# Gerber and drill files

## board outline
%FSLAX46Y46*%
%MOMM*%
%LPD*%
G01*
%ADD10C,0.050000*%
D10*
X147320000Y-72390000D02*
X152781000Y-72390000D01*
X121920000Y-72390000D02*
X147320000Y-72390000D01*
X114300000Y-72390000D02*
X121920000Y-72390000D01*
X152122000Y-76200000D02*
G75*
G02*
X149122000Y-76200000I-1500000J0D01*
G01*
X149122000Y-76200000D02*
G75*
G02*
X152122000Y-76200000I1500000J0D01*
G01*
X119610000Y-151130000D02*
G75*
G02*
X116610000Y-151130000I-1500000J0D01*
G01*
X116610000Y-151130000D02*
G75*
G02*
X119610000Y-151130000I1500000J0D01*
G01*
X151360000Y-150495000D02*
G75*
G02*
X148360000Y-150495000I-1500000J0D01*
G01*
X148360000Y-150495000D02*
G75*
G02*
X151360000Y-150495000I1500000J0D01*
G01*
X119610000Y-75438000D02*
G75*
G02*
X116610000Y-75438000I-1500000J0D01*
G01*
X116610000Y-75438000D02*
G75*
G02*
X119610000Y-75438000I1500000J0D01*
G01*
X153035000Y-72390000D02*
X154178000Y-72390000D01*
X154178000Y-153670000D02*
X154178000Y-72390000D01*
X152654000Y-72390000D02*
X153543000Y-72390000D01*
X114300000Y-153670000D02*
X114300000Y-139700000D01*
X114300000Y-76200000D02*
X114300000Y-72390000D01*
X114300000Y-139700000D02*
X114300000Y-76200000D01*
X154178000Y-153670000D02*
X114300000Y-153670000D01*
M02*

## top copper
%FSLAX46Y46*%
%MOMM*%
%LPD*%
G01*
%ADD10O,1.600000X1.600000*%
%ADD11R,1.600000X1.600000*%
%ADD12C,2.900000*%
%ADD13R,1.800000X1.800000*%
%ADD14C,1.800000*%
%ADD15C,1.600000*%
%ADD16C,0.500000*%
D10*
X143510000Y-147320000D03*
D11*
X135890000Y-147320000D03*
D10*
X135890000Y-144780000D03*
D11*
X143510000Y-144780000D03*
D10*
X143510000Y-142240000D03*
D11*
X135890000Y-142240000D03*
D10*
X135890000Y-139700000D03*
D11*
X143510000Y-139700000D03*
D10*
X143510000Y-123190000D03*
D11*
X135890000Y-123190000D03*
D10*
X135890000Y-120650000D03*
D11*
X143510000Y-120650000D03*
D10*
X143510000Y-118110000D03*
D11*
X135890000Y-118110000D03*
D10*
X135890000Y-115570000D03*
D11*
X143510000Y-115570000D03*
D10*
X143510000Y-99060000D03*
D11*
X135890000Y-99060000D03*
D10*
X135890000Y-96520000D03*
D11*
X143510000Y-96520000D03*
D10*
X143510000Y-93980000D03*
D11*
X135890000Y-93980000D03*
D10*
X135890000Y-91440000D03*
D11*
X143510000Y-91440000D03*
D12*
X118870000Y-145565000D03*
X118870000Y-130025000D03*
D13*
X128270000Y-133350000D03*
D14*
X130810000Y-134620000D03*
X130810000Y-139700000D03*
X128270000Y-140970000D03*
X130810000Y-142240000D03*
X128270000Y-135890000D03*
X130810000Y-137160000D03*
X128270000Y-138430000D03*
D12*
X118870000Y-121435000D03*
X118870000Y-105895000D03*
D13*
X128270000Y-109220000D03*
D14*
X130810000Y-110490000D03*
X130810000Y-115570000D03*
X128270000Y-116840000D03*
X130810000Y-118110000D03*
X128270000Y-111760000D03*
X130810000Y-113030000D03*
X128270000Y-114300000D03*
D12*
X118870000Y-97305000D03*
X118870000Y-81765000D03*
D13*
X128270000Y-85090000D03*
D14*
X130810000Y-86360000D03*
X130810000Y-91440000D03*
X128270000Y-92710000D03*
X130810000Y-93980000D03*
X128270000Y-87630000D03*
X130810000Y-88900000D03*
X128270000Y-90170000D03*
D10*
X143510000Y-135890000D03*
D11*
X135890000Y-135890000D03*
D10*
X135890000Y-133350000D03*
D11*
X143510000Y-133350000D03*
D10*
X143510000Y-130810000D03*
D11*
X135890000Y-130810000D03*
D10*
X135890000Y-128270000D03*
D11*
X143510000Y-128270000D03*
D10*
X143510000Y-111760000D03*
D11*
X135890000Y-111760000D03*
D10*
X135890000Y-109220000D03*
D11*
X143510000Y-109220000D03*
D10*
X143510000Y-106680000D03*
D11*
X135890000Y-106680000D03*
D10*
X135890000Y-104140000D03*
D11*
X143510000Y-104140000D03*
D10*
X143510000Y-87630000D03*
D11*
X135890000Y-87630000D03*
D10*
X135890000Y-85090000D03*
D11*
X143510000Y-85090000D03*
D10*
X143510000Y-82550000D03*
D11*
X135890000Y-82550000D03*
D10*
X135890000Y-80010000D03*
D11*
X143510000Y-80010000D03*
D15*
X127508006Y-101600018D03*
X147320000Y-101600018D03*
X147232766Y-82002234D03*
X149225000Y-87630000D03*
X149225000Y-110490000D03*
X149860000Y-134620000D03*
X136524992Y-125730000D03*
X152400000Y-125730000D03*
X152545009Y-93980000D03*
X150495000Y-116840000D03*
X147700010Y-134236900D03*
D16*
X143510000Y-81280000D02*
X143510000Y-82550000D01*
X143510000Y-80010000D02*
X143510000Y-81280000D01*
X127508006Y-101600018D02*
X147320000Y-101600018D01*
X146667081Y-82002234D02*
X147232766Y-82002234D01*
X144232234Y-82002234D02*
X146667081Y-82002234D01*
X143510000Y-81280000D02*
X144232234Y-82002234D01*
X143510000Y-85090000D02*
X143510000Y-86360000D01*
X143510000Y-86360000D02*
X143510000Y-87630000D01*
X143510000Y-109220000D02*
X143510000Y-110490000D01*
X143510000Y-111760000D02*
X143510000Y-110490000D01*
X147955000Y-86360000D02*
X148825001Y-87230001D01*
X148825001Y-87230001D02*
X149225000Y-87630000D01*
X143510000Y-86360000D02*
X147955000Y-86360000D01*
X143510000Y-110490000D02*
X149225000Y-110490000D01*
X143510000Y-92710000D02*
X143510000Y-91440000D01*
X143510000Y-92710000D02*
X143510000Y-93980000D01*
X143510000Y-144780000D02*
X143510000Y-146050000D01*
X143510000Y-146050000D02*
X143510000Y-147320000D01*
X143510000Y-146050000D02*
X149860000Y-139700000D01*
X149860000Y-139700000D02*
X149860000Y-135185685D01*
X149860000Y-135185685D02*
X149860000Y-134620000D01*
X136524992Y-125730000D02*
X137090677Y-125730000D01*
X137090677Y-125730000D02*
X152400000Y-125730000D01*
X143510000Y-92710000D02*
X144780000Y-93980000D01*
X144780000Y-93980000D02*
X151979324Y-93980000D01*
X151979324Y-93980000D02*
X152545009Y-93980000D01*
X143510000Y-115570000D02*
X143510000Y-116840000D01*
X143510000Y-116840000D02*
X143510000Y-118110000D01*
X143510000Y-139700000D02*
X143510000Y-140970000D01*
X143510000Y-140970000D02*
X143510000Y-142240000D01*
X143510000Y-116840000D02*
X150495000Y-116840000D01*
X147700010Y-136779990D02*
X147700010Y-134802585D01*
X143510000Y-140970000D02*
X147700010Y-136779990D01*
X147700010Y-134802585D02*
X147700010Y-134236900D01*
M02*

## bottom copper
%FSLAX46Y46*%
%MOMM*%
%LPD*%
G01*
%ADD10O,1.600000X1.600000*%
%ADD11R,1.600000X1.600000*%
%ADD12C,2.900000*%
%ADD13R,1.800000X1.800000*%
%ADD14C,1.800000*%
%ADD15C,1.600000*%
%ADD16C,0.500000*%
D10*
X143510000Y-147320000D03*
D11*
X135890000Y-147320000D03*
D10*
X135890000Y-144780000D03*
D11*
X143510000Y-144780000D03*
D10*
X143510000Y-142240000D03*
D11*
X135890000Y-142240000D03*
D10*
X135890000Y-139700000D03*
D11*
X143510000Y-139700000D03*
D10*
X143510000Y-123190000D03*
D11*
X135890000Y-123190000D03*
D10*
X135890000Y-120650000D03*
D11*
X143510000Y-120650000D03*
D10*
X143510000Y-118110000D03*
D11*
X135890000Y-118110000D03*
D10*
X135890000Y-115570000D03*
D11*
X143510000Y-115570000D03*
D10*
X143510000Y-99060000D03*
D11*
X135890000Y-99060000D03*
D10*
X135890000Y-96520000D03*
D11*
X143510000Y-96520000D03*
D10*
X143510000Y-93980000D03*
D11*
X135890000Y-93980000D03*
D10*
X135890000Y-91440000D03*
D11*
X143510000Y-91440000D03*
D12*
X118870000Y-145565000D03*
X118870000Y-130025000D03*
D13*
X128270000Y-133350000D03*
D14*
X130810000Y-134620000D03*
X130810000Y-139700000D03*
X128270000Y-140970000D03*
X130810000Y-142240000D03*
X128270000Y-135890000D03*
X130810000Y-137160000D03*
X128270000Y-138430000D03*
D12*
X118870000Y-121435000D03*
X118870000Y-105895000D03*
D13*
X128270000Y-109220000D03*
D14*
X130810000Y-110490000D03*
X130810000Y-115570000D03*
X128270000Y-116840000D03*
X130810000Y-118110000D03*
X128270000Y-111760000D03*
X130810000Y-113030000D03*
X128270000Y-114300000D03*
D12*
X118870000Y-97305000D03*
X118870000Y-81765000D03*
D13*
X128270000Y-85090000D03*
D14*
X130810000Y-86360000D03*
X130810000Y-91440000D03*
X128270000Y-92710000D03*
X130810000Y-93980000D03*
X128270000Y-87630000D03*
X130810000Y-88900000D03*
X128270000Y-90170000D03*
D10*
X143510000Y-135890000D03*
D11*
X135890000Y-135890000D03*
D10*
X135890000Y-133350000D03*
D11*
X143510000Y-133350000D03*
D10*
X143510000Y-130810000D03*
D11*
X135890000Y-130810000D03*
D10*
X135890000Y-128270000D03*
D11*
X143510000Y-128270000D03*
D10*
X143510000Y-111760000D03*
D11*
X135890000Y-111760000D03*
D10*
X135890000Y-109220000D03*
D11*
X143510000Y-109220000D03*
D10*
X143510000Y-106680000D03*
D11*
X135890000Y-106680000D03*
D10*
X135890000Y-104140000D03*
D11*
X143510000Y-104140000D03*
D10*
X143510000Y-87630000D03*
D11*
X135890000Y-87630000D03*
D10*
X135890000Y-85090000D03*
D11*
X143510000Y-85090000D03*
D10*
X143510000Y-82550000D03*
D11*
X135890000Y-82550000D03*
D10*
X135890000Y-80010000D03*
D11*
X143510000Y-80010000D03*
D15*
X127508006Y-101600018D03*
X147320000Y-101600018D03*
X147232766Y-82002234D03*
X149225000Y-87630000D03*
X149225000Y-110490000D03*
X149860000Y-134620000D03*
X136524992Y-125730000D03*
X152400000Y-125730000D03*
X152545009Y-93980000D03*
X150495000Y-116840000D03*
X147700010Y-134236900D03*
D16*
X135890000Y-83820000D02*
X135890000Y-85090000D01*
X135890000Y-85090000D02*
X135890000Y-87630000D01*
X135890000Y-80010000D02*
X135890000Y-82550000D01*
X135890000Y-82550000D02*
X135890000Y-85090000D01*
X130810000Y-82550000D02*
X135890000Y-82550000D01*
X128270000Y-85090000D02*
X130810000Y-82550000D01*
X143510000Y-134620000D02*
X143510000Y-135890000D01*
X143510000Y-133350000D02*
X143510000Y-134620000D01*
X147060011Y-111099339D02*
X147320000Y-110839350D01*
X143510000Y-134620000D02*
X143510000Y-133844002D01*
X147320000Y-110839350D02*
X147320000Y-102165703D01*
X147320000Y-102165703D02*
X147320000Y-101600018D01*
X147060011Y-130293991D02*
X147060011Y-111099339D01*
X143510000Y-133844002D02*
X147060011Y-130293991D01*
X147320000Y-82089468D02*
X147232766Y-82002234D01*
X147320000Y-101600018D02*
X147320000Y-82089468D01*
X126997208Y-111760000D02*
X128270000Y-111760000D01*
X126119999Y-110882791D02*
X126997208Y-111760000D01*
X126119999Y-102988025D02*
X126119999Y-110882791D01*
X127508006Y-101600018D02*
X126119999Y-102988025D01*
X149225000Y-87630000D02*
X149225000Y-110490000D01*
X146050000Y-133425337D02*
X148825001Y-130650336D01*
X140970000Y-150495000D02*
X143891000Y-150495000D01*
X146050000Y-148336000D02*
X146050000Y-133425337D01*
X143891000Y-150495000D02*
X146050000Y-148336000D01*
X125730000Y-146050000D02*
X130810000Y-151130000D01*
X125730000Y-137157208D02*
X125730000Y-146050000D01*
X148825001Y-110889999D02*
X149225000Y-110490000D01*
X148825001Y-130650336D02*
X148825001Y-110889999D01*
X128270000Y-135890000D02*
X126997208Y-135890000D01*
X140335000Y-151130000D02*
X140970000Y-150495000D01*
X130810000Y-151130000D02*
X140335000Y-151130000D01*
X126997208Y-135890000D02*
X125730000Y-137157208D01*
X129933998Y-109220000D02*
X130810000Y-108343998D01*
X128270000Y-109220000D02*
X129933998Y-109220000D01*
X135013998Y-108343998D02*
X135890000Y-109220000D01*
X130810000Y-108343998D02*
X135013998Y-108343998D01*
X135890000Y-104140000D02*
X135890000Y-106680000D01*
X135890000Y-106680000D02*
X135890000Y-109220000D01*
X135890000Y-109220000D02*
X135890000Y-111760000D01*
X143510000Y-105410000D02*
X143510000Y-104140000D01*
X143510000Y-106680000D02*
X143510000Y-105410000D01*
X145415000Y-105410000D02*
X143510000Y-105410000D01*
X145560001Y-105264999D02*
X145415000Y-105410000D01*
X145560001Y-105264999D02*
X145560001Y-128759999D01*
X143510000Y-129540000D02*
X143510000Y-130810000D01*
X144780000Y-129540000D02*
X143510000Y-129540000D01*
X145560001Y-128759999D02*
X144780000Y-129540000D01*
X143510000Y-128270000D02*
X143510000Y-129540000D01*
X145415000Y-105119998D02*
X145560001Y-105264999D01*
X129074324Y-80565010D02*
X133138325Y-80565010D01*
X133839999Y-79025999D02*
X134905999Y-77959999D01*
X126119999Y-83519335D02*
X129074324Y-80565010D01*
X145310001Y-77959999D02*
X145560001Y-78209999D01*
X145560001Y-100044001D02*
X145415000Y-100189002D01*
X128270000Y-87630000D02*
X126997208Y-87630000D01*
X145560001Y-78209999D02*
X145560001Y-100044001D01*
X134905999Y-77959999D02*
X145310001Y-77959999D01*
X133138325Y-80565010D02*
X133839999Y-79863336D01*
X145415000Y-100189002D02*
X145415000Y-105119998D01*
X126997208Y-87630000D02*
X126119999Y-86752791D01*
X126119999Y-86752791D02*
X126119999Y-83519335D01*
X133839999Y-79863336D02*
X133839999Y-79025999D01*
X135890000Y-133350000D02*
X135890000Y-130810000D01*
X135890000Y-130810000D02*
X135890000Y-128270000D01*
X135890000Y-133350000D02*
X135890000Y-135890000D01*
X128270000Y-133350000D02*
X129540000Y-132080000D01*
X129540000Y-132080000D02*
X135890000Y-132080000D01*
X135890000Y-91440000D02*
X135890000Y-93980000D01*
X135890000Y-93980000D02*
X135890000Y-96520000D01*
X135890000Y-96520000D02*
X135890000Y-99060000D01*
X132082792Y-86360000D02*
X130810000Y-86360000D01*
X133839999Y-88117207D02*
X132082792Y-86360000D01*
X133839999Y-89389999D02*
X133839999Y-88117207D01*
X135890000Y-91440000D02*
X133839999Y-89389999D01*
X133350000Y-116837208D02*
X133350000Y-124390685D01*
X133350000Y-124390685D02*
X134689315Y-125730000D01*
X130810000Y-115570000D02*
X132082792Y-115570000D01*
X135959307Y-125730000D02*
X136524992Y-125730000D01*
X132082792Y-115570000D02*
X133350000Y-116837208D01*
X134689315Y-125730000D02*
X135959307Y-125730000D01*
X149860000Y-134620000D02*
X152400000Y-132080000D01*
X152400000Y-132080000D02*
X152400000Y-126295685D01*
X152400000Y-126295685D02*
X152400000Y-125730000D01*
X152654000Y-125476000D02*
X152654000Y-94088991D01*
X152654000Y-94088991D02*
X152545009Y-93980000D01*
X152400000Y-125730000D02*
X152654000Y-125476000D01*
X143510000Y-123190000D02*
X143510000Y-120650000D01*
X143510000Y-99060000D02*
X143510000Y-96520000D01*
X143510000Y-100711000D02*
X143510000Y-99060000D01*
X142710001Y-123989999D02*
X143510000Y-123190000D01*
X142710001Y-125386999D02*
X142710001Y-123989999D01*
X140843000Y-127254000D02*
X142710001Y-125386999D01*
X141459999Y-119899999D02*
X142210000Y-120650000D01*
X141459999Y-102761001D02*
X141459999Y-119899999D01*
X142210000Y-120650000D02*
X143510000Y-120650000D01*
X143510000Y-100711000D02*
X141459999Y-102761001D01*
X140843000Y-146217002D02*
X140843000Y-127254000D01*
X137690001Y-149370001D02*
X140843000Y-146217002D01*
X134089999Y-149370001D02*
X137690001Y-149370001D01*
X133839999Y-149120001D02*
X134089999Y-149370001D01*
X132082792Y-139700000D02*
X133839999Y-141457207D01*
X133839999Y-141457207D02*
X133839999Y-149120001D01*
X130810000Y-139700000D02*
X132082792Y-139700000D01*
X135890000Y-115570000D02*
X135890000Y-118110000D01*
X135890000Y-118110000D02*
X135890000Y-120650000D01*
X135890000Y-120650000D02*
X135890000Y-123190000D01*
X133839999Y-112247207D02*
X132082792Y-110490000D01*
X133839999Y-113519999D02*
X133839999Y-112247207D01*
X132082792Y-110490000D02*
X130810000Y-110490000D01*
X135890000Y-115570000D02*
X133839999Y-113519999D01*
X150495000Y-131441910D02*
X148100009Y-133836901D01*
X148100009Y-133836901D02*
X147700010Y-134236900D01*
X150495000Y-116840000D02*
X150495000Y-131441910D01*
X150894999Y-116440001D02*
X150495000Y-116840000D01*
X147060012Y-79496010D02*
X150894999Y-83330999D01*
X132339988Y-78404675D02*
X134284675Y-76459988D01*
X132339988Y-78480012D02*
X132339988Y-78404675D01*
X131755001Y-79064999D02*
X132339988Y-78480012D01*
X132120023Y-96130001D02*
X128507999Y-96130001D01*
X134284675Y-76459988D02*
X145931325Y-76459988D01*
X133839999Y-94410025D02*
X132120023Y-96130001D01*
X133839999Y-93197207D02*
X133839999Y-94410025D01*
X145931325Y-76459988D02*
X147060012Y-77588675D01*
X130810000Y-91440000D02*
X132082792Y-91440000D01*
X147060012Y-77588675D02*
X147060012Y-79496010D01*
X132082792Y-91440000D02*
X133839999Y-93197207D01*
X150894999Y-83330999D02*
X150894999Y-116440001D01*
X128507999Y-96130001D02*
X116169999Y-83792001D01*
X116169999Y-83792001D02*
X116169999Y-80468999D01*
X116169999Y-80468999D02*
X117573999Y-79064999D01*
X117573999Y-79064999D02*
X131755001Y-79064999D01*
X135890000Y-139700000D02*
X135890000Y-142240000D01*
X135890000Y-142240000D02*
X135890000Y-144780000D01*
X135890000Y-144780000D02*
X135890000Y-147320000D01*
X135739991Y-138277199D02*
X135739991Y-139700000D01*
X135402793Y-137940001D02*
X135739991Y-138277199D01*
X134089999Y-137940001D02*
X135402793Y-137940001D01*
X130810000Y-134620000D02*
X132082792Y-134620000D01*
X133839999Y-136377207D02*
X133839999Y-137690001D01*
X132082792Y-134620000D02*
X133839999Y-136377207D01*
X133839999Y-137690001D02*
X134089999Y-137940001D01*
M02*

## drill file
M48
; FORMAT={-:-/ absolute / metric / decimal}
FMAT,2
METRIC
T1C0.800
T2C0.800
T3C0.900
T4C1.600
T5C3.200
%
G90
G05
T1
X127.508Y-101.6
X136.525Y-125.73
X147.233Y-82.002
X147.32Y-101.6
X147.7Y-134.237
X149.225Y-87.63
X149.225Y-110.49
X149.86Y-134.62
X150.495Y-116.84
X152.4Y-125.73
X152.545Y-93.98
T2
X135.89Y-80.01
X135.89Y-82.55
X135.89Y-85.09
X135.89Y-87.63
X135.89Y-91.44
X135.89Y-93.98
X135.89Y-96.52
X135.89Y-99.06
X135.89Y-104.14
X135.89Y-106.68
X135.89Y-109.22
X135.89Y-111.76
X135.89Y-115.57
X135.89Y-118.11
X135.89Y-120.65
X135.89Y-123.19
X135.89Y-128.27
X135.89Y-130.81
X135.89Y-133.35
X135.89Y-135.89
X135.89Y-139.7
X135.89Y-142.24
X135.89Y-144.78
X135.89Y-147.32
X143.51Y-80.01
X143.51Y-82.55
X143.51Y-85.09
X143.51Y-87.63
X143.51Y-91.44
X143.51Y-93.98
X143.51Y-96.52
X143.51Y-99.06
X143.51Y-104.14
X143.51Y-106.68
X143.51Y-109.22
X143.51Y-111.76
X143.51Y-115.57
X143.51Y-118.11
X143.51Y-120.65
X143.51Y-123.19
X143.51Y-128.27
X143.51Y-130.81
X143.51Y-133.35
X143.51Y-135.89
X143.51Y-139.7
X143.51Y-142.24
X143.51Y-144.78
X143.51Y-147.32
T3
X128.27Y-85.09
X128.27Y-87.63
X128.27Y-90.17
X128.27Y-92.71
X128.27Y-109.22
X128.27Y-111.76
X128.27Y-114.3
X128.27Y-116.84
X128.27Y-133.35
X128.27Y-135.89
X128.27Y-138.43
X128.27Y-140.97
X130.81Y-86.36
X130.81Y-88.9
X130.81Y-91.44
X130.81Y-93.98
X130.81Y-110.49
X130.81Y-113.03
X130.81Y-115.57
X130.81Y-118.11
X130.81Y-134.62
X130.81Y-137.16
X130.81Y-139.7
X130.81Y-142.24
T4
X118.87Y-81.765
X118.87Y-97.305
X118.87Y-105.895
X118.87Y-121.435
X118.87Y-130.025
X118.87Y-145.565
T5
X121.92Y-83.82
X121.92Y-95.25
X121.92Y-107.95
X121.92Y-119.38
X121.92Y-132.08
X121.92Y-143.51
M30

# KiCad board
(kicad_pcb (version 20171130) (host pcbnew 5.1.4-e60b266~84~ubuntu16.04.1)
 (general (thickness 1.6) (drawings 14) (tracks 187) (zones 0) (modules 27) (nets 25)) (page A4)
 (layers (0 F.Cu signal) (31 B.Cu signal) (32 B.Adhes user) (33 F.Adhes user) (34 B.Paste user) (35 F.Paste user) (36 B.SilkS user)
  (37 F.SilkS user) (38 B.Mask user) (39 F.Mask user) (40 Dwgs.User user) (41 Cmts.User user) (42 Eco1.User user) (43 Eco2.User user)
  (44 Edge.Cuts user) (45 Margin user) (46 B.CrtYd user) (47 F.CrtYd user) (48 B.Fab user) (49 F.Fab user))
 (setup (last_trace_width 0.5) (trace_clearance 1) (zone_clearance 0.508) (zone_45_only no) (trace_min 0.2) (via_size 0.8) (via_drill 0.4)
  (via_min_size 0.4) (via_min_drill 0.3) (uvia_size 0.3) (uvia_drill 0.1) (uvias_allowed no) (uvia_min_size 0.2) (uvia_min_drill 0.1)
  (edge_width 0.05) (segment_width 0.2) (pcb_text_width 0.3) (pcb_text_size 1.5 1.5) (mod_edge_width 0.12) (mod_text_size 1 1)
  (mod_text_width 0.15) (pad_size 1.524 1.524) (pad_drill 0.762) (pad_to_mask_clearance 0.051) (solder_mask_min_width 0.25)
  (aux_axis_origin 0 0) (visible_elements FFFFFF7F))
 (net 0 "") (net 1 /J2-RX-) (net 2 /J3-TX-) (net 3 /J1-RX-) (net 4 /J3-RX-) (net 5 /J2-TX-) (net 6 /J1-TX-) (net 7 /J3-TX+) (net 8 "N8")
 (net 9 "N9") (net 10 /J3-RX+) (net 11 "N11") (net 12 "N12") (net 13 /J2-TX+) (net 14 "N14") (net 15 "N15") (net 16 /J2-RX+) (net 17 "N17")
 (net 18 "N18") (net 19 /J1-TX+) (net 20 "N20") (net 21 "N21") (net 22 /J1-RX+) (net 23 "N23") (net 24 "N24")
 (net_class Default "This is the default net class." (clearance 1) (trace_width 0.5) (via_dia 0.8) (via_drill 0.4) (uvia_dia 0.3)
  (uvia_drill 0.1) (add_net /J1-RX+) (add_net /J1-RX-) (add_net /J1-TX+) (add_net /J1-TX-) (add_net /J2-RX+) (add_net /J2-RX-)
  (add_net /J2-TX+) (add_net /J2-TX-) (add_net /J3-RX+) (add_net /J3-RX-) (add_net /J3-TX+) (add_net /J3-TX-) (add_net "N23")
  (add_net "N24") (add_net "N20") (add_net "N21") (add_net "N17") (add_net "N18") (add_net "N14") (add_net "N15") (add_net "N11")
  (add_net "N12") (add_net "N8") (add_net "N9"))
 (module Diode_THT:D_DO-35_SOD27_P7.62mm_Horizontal (layer F.Cu) (at 135.89 147.32)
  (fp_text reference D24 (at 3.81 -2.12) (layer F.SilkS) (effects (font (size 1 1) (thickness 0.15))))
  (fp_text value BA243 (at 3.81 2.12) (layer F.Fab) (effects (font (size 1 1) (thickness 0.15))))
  (pad 2 thru_hole oval (at 7.62 0) (size 1.6 1.6) (drill 0.8) (layers *.Cu *.Mask) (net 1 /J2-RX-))
  (pad 1 thru_hole rect (at 0 0) (size 1.6 1.6) (drill 0.8) (layers *.Cu *.Mask) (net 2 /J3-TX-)))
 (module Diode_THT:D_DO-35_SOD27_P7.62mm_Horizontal (layer F.Cu) (at 143.51 144.78 180)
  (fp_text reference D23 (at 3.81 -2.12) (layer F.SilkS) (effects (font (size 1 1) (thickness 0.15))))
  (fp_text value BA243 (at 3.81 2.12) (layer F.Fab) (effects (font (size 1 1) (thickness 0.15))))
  (pad 2 thru_hole oval (at 7.62 0 180) (size 1.6 1.6) (drill 0.8) (layers *.Cu *.Mask) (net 2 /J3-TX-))
  (pad 1 thru_hole rect (at 0 0 180) (size 1.6 1.6) (drill 0.8) (layers *.Cu *.Mask) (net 1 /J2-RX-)))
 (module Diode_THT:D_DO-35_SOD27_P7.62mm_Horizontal (layer F.Cu) (at 135.89 142.24)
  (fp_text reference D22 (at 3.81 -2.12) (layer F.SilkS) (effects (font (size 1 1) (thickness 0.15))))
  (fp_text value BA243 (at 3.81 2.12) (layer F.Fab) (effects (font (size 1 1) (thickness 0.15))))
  (pad 2 thru_hole oval (at 7.62 0) (size 1.6 1.6) (drill 0.8) (layers *.Cu *.Mask) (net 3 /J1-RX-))
  (pad 1 thru_hole rect (at 0 0) (size 1.6 1.6) (drill 0.8) (layers *.Cu *.Mask) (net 2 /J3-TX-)))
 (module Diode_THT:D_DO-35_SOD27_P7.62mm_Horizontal (layer F.Cu) (at 143.51 139.7 180)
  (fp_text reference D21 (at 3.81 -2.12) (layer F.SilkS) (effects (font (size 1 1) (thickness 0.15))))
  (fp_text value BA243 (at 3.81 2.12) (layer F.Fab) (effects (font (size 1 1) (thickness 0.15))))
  (pad 2 thru_hole oval (at 7.62 0 180) (size 1.6 1.6) (drill 0.8) (layers *.Cu *.Mask) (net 2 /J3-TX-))
  (pad 1 thru_hole rect (at 0 0 180) (size 1.6 1.6) (drill 0.8) (layers *.Cu *.Mask) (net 3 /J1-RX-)))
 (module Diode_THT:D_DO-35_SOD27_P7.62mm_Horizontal (layer F.Cu) (at 135.89 123.19)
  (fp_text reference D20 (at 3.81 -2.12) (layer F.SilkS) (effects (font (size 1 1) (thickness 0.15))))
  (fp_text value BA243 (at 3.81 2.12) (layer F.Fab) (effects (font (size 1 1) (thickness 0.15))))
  (pad 2 thru_hole oval (at 7.62 0) (size 1.6 1.6) (drill 0.8) (layers *.Cu *.Mask) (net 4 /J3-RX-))
  (pad 1 thru_hole rect (at 0 0) (size 1.6 1.6) (drill 0.8) (layers *.Cu *.Mask) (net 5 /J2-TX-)))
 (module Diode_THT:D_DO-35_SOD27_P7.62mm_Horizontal (layer F.Cu) (at 143.51 120.65 180)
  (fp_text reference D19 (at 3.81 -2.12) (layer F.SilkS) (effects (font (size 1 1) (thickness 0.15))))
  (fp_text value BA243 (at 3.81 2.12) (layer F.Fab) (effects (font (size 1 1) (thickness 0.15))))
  (pad 2 thru_hole oval (at 7.62 0 180) (size 1.6 1.6) (drill 0.8) (layers *.Cu *.Mask) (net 5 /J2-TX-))
  (pad 1 thru_hole rect (at 0 0 180) (size 1.6 1.6) (drill 0.8) (layers *.Cu *.Mask) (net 4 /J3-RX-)))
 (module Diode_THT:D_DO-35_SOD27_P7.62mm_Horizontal (layer F.Cu) (at 135.89 118.11)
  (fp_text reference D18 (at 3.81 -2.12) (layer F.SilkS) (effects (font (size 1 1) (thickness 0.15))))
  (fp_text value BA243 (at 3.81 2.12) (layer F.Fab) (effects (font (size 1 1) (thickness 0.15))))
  (pad 2 thru_hole oval (at 7.62 0) (size 1.6 1.6) (drill 0.8) (layers *.Cu *.Mask) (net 3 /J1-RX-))
  (pad 1 thru_hole rect (at 0 0) (size 1.6 1.6) (drill 0.8) (layers *.Cu *.Mask) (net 5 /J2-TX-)))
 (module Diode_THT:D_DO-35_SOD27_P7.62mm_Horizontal (layer F.Cu) (at 143.51 115.57 180)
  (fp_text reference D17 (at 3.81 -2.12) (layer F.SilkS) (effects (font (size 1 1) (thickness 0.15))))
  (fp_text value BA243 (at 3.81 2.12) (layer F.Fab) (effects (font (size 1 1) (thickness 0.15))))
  (pad 2 thru_hole oval (at 7.62 0 180) (size 1.6 1.6) (drill 0.8) (layers *.Cu *.Mask) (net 5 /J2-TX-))
  (pad 1 thru_hole rect (at 0 0 180) (size 1.6 1.6) (drill 0.8) (layers *.Cu *.Mask) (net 3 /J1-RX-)))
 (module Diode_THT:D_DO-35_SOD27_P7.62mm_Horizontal (layer F.Cu) (at 135.89 99.06)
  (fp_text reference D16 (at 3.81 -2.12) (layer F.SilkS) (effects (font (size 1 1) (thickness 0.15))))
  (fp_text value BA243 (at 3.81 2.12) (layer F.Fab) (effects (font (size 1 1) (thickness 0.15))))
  (pad 2 thru_hole oval (at 7.62 0) (size 1.6 1.6) (drill 0.8) (layers *.Cu *.Mask) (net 4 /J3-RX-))
  (pad 1 thru_hole rect (at 0 0) (size 1.6 1.6) (drill 0.8) (layers *.Cu *.Mask) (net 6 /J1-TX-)))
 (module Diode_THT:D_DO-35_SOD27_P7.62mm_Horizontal (layer F.Cu) (at 143.51 96.52 180)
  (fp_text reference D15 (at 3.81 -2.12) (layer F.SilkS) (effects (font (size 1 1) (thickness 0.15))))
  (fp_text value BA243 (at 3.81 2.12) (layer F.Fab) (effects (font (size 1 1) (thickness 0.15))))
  (pad 2 thru_hole oval (at 7.62 0 180) (size 1.6 1.6) (drill 0.8) (layers *.Cu *.Mask) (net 6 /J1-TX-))
  (pad 1 thru_hole rect (at 0 0 180) (size 1.6 1.6) (drill 0.8) (layers *.Cu *.Mask) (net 4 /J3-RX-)))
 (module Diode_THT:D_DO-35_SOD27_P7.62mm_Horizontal (layer F.Cu) (at 135.89 93.98)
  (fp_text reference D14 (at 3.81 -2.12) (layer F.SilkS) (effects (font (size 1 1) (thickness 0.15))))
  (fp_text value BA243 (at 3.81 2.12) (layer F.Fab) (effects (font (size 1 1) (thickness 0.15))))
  (pad 2 thru_hole oval (at 7.62 0) (size 1.6 1.6) (drill 0.8) (layers *.Cu *.Mask) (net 1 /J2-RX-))
  (pad 1 thru_hole rect (at 0 0) (size 1.6 1.6) (drill 0.8) (layers *.Cu *.Mask) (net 6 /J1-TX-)))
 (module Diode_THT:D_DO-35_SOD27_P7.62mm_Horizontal (layer F.Cu) (at 143.51 91.44 180)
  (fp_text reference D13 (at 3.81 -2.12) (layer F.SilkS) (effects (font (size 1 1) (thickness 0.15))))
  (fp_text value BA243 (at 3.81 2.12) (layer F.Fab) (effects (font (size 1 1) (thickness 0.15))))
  (pad 2 thru_hole oval (at 7.62 0 180) (size 1.6 1.6) (drill 0.8) (layers *.Cu *.Mask) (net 6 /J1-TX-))
  (pad 1 thru_hole rect (at 0 0 180) (size 1.6 1.6) (drill 0.8) (layers *.Cu *.Mask) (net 1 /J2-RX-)))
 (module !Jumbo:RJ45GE (layer F.Cu) (at 123.19 138.43 270)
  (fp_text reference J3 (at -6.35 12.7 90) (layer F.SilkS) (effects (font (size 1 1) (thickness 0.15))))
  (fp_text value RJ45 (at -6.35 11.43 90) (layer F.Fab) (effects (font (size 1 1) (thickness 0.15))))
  (pad 10 thru_hole circle (at 7.135 4.32 270) (size 2.9 2.9) (drill 1.6) (layers *.Cu *.Mask))
  (pad 9 thru_hole circle (at -8.405 4.32 270) (size 2.9 2.9) (drill 1.6) (layers *.Cu *.Mask))
  (pad 1 thru_hole rect (at -5.08 -5.08 270) (size 1.8 1.8) (drill 0.9) (layers *.Cu *.Mask) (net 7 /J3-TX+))
  (pad 2 thru_hole circle (at -3.81 -7.62 270) (size 1.8 1.8) (drill 0.9) (layers *.Cu *.Mask) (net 2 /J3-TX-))
  (pad 6 thru_hole circle (at 1.27 -7.62 270) (size 1.8 1.8) (drill 0.9) (layers *.Cu *.Mask) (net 4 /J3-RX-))
  (pad 7 thru_hole circle (at 2.54 -5.08 270) (size 1.8 1.8) (drill 0.9) (layers *.Cu *.Mask) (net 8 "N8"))
  (pad 8 thru_hole circle (at 3.81 -7.62 270) (size 1.8 1.8) (drill 0.9) (layers *.Cu *.Mask) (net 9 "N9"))
  (pad "" np_thru_hole circle (at 5.08 1.27 270) (size 3.2 3.2) (drill 3.2) (layers *.Cu *.Mask))
  (pad "" np_thru_hole circle (at -6.35 1.27 270) (size 3.2 3.2) (drill 3.2) (layers *.Cu *.Mask))
  (pad 3 thru_hole circle (at -2.54 -5.08 270) (size 1.8 1.8) (drill 0.9) (layers *.Cu *.Mask) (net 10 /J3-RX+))
  (pad 4 thru_hole circle (at -1.27 -7.62 270) (size 1.8 1.8) (drill 0.9) (layers *.Cu *.Mask) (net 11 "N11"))
  (pad 5 thru_hole circle (at 0 -5.08 270) (size 1.8 1.8) (drill 0.9) (layers *.Cu *.Mask) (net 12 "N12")))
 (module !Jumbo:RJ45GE (layer F.Cu) (at 123.19 114.3 270)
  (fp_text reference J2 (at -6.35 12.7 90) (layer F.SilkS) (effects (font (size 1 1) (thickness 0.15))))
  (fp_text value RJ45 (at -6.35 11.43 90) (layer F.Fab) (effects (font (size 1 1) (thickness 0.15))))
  (pad 10 thru_hole circle (at 7.135 4.32 270) (size 2.9 2.9) (drill 1.6) (layers *.Cu *.Mask))
  (pad 9 thru_hole circle (at -8.405 4.32 270) (size 2.9 2.9) (drill 1.6) (layers *.Cu *.Mask))
  (pad 1 thru_hole rect (at -5.08 -5.08 270) (size 1.8 1.8) (drill 0.9) (layers *.Cu *.Mask) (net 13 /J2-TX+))
  (pad 2 thru_hole circle (at -3.81 -7.62 270) (size 1.8 1.8) (drill 0.9) (layers *.Cu *.Mask) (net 5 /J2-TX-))
  (pad 6 thru_hole circle (at 1.27 -7.62 270) (size 1.8 1.8) (drill 0.9) (layers *.Cu *.Mask) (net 1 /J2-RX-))
  (pad 7 thru_hole circle (at 2.54 -5.08 270) (size 1.8 1.8) (drill 0.9) (layers *.Cu *.Mask) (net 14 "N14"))
  (pad 8 thru_hole circle (at 3.81 -7.62 270) (size 1.8 1.8) (drill 0.9) (layers *.Cu *.Mask) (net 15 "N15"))
  (pad "" np_thru_hole circle (at 5.08 1.27 270) (size 3.2 3.2) (drill 3.2) (layers *.Cu *.Mask))
  (pad "" np_thru_hole circle (at -6.35 1.27 270) (size 3.2 3.2) (drill 3.2) (layers *.Cu *.Mask))
  (pad 3 thru_hole circle (at -2.54 -5.08 270) (size 1.8 1.8) (drill 0.9) (layers *.Cu *.Mask) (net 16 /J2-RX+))
  (pad 4 thru_hole circle (at -1.27 -7.62 270) (size 1.8 1.8) (drill 0.9) (layers *.Cu *.Mask) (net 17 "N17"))
  (pad 5 thru_hole circle (at 0 -5.08 270) (size 1.8 1.8) (drill 0.9) (layers *.Cu *.Mask) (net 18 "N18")))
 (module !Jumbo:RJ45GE (layer F.Cu) (at 123.19 90.17 270)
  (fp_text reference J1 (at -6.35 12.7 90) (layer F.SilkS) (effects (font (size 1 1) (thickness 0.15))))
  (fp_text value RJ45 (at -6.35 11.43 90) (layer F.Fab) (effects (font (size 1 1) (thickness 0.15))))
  (pad 10 thru_hole circle (at 7.135 4.32 270) (size 2.9 2.9) (drill 1.6) (layers *.Cu *.Mask))
  (pad 9 thru_hole circle (at -8.405 4.32 270) (size 2.9 2.9) (drill 1.6) (layers *.Cu *.Mask))
  (pad 1 thru_hole rect (at -5.08 -5.08 270) (size 1.8 1.8) (drill 0.9) (layers *.Cu *.Mask) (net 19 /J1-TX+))
  (pad 2 thru_hole circle (at -3.81 -7.62 270) (size 1.8 1.8) (drill 0.9) (layers *.Cu *.Mask) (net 6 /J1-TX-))
  (pad 6 thru_hole circle (at 1.27 -7.62 270) (size 1.8 1.8) (drill 0.9) (layers *.Cu *.Mask) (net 3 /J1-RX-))
  (pad 7 thru_hole circle (at 2.54 -5.08 270) (size 1.8 1.8) (drill 0.9) (layers *.Cu *.Mask) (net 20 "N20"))
  (pad 8 thru_hole circle (at 3.81 -7.62 270) (size 1.8 1.8) (drill 0.9) (layers *.Cu *.Mask) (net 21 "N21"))
  (pad "" np_thru_hole circle (at 5.08 1.27 270) (size 3.2 3.2) (drill 3.2) (layers *.Cu *.Mask))
  (pad "" np_thru_hole circle (at -6.35 1.27 270) (size 3.2 3.2) (drill 3.2) (layers *.Cu *.Mask))
  (pad 3 thru_hole circle (at -2.54 -5.08 270) (size 1.8 1.8) (drill 0.9) (layers *.Cu *.Mask) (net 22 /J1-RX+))
  (pad 4 thru_hole circle (at -1.27 -7.62 270) (size 1.8 1.8) (drill 0.9) (layers *.Cu *.Mask) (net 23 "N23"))
  (pad 5 thru_hole circle (at 0 -5.08 270) (size 1.8 1.8) (drill 0.9) (layers *.Cu *.Mask) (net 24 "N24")))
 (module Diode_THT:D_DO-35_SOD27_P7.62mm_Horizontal (layer F.Cu) (at 135.89 135.89)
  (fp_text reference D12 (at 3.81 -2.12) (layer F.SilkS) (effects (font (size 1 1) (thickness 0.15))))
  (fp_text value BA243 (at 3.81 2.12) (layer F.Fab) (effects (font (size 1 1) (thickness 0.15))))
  (pad 2 thru_hole oval (at 7.62 0) (size 1.6 1.6) (drill 0.8) (layers *.Cu *.Mask) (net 16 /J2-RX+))
  (pad 1 thru_hole rect (at 0 0) (size 1.6 1.6) (drill 0.8) (layers *.Cu *.Mask) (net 7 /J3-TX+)))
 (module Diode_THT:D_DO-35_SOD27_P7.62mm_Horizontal (layer F.Cu) (at 143.51 133.35 180)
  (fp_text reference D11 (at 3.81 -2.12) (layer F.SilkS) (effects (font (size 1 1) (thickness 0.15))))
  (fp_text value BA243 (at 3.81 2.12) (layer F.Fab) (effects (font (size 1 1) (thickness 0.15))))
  (pad 2 thru_hole oval (at 7.62 0 180) (size 1.6 1.6) (drill 0.8) (layers *.Cu *.Mask) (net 7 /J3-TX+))
  (pad 1 thru_hole rect (at 0 0 180) (size 1.6 1.6) (drill 0.8) (layers *.Cu *.Mask) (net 16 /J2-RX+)))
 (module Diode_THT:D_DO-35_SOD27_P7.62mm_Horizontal (layer F.Cu) (at 135.89 130.81)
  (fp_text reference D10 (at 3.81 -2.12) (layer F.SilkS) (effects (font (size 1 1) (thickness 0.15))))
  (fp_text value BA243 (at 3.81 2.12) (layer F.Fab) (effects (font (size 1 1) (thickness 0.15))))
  (pad 2 thru_hole oval (at 7.62 0) (size 1.6 1.6) (drill 0.8) (layers *.Cu *.Mask) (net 22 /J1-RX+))
  (pad 1 thru_hole rect (at 0 0) (size 1.6 1.6) (drill 0.8) (layers *.Cu *.Mask) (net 7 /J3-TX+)))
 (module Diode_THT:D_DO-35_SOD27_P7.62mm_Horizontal (layer F.Cu) (at 143.51 128.27 180)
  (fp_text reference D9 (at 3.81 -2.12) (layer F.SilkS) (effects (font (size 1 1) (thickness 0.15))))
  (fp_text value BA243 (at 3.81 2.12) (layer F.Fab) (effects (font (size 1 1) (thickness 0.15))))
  (pad 2 thru_hole oval (at 7.62 0 180) (size 1.6 1.6) (drill 0.8) (layers *.Cu *.Mask) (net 7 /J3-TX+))
  (pad 1 thru_hole rect (at 0 0 180) (size 1.6 1.6) (drill 0.8) (layers *.Cu *.Mask) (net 22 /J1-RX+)))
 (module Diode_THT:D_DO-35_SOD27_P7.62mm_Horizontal (layer F.Cu) (at 135.89 111.76)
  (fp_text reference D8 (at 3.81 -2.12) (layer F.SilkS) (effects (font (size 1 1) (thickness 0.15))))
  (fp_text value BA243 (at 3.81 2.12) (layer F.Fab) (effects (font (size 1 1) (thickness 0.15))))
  (pad 2 thru_hole oval (at 7.62 0) (size 1.6 1.6) (drill 0.8) (layers *.Cu *.Mask) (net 10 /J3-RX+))
  (pad 1 thru_hole rect (at 0 0) (size 1.6 1.6) (drill 0.8) (layers *.Cu *.Mask) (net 13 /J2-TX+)))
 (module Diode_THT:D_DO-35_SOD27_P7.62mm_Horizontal (layer F.Cu) (at 143.51 109.22 180)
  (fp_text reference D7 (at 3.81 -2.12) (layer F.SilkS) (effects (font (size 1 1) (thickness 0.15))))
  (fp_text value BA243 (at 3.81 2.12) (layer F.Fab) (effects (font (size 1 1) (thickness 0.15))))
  (pad 2 thru_hole oval (at 7.62 0 180) (size 1.6 1.6) (drill 0.8) (layers *.Cu *.Mask) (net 13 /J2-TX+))
  (pad 1 thru_hole rect (at 0 0 180) (size 1.6 1.6) (drill 0.8) (layers *.Cu *.Mask) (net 10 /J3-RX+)))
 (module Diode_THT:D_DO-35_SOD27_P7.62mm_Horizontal (layer F.Cu) (at 135.89 106.68)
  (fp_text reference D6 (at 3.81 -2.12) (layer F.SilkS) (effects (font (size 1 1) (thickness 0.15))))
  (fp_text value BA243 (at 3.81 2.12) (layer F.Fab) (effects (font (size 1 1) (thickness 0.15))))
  (pad 2 thru_hole oval (at 7.62 0) (size 1.6 1.6) (drill 0.8) (layers *.Cu *.Mask) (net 22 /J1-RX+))
  (pad 1 thru_hole rect (at 0 0) (size 1.6 1.6) (drill 0.8) (layers *.Cu *.Mask) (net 13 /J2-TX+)))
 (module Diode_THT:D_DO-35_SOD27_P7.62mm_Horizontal (layer F.Cu) (at 143.51 104.14 180)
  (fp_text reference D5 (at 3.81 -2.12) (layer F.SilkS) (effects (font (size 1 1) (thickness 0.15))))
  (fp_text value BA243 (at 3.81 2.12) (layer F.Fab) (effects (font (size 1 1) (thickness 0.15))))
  (pad 2 thru_hole oval (at 7.62 0 180) (size 1.6 1.6) (drill 0.8) (layers *.Cu *.Mask) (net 13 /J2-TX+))
  (pad 1 thru_hole rect (at 0 0 180) (size 1.6 1.6) (drill 0.8) (layers *.Cu *.Mask) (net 22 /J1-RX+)))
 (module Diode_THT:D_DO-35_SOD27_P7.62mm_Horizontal (layer F.Cu) (at 135.89 87.63)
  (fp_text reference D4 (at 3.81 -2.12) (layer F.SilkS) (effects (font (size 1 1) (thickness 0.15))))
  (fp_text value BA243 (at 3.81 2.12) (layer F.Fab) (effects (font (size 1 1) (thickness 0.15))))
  (pad 2 thru_hole oval (at 7.62 0) (size 1.6 1.6) (drill 0.8) (layers *.Cu *.Mask) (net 10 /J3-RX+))
  (pad 1 thru_hole rect (at 0 0) (size 1.6 1.6) (drill 0.8) (layers *.Cu *.Mask) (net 19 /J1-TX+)))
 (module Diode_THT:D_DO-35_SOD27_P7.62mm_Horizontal (layer F.Cu) (at 143.51 85.09 180)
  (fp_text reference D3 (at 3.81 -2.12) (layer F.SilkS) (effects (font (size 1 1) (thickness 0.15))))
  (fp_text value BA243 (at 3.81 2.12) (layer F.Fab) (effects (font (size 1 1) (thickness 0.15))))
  (pad 2 thru_hole oval (at 7.62 0 180) (size 1.6 1.6) (drill 0.8) (layers *.Cu *.Mask) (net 19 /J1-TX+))
  (pad 1 thru_hole rect (at 0 0 180) (size 1.6 1.6) (drill 0.8) (layers *.Cu *.Mask) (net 10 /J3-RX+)))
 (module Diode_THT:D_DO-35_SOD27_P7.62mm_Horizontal (layer F.Cu) (at 135.89 82.55)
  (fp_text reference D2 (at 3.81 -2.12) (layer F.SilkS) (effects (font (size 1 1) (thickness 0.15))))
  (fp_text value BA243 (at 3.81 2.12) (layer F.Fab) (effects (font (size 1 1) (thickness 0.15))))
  (pad 2 thru_hole oval (at 7.62 0) (size 1.6 1.6) (drill 0.8) (layers *.Cu *.Mask) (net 16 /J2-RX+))
  (pad 1 thru_hole rect (at 0 0) (size 1.6 1.6) (drill 0.8) (layers *.Cu *.Mask) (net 19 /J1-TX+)))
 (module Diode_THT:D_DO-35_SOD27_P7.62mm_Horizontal (layer F.Cu) (at 143.51 80.01 180)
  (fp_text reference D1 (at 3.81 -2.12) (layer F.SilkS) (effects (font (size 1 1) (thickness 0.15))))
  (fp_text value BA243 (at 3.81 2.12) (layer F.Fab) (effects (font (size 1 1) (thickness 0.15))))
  (pad 2 thru_hole oval (at 7.62 0 180) (size 1.6 1.6) (drill 0.8) (layers *.Cu *.Mask) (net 19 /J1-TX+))
  (pad 1 thru_hole rect (at 0 0 180) (size 1.6 1.6) (drill 0.8) (layers *.Cu *.Mask) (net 16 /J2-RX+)))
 (gr_line (start 147.32 72.39) (end 152.781 72.39) (layer Edge.Cuts) (width 0.05))
 (gr_line (start 121.92 72.39) (end 147.32 72.39) (layer Edge.Cuts) (width 0.05))
 (gr_line (start 114.3 72.39) (end 121.92 72.39) (layer Edge.Cuts) (width 0.05))
 (gr_circle (center 150.622 76.2) (end 152.122 76.2) (layer Edge.Cuts) (width 0.05))
 (gr_circle (center 118.11 151.13) (end 119.61 151.13) (layer Edge.Cuts) (width 0.05))
 (gr_circle (center 149.86 150.495) (end 151.36 150.495) (layer Edge.Cuts) (width 0.05))
 (gr_circle (center 118.11 75.438) (end 119.61 75.438) (layer Edge.Cuts) (width 0.05))
 (gr_line (start 153.035 72.39) (end 154.178 72.39) (layer Edge.Cuts) (width 0.05))
 (gr_line (start 154.178 153.67) (end 154.178 72.39) (layer Edge.Cuts) (width 0.05))
 (gr_line (start 152.654 72.39) (end 153.543 72.39) (layer Edge.Cuts) (width 0.05))
 (gr_line (start 114.3 153.67) (end 114.3 139.7) (layer Edge.Cuts) (width 0.05))
 (gr_line (start 114.3 76.2) (end 114.3 72.39) (layer Edge.Cuts) (width 0.05))
 (gr_line (start 114.3 139.7) (end 114.3 76.2) (layer Edge.Cuts) (width 0.05))
 (gr_line (start 154.178 153.67) (end 114.3 153.67) (layer Edge.Cuts) (width 0.05))
 (segment (start 135.89 83.82) (end 135.89 85.09) (width 0.5) (layer B.Cu) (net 19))
 (segment (start 135.89 85.09) (end 135.89 87.63) (width 0.5) (layer B.Cu) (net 19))
 (segment (start 135.89 80.01) (end 135.89 82.55) (width 0.5) (layer B.Cu) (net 19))
 (segment (start 135.89 82.55) (end 135.89 85.09) (width 0.5) (layer B.Cu) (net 19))
 (segment (start 130.81 82.55) (end 135.89 82.55) (width 0.5) (layer B.Cu) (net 19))
 (segment (start 128.27 85.09) (end 130.81 82.55) (width 0.5) (layer B.Cu) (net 19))
 (segment (start 143.51 134.62) (end 143.51 135.89) (width 0.5) (layer B.Cu) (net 16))
 (segment (start 143.51 133.35) (end 143.51 134.62) (width 0.5) (layer B.Cu) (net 16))
 (via (at 127.508006 101.600018) (size 1.6) (drill 0.8) (layers F.Cu B.Cu) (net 16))
 (segment (start 143.51 81.28) (end 143.51 82.55) (width 0.5) (layer F.Cu) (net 16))
 (segment (start 143.51 80.01) (end 143.51 81.28) (width 0.5) (layer F.Cu) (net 16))
 (via (at 147.32 101.600018) (size 1.6) (drill 0.8) (layers F.Cu B.Cu) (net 16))
 (segment (start 127.508006 101.600018) (end 147.32 101.600018) (width 0.5) (layer F.Cu) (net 16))
 (segment (start 147.060011 111.099339) (end 147.32 110.83935) (width 0.5) (layer B.Cu) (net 16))
 (segment (start 143.51 134.62) (end 143.51 133.844002) (width 0.5) (layer B.Cu) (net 16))
 (segment (start 147.32 110.83935) (end 147.32 102.165703) (width 0.5) (layer B.Cu) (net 16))
 (segment (start 147.32 102.165703) (end 147.32 101.600018) (width 0.5) (layer B.Cu) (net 16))
 (segment (start 147.060011 130.293991) (end 147.060011 111.099339) (width 0.5) (layer B.Cu) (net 16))
 (segment (start 143.51 133.844002) (end 147.060011 130.293991) (width 0.5) (layer B.Cu) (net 16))
 (segment (start 147.32 82.089468) (end 147.232766 82.002234) (width 0.5) (layer B.Cu) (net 16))
 (via (at 147.232766 82.002234) (size 1.6) (drill 0.8) (layers F.Cu B.Cu) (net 16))
 (segment (start 147.32 101.600018) (end 147.32 82.089468) (width 0.5) (layer B.Cu) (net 16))
 (segment (start 146.667081 82.002234) (end 147.232766 82.002234) (width 0.5) (layer F.Cu) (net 16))
 (segment (start 144.232234 82.002234) (end 146.667081 82.002234) (width 0.5) (layer F.Cu) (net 16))
 (segment (start 143.51 81.28) (end 144.232234 82.002234) (width 0.5) (layer F.Cu) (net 16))
 (segment (start 126.997208 111.76) (end 128.27 111.76) (width 0.5) (layer B.Cu) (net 16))
 (segment (start 126.119999 110.882791) (end 126.997208 111.76) (width 0.5) (layer B.Cu) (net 16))
 (segment (start 126.119999 102.988025) (end 126.119999 110.882791) (width 0.5) (layer B.Cu) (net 16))
 (segment (start 127.508006 101.600018) (end 126.119999 102.988025) (width 0.5) (layer B.Cu) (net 16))
 (segment (start 143.51 85.09) (end 143.51 86.36) (width 0.5) (layer F.Cu) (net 10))
 (segment (start 143.51 86.36) (end 143.51 87.63) (width 0.5) (layer F.Cu) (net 10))
 (segment (start 143.51 109.22) (end 143.51 110.49) (width 0.5) (layer F.Cu) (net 10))
 (segment (start 143.51 111.76) (end 143.51 110.49) (width 0.5) (layer F.Cu) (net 10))
 (segment (start 147.955 86.36) (end 148.825001 87.230001) (width 0.5) (layer F.Cu) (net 10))
 (segment (start 148.825001 87.230001) (end 149.225 87.63) (width 0.5) (layer F.Cu) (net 10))
 (segment (start 143.51 86.36) (end 147.955 86.36) (width 0.5) (layer F.Cu) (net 10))
 (via (at 149.225 87.63) (size 1.6) (drill 0.8) (layers F.Cu B.Cu) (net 10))
 (segment (start 149.225 87.63) (end 149.225 110.49) (width 0.5) (layer B.Cu) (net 10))
 (segment (start 143.51 110.49) (end 149.225 110.49) (width 0.5) (layer F.Cu) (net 10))
 (via (at 149.225 110.49) (size 1.6) (drill 0.8) (layers F.Cu B.Cu) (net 10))
 (segment (start 146.05 133.425337) (end 148.825001 130.650336) (width 0.5) (layer B.Cu) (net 10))
 (segment (start 140.97 150.495) (end 143.891 150.495) (width 0.5) (layer B.Cu) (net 10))
 (segment (start 146.05 148.336) (end 146.05 133.425337) (width 0.5) (layer B.Cu) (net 10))
 (segment (start 143.891 150.495) (end 146.05 148.336) (width 0.5) (layer B.Cu) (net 10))
 (segment (start 125.73 146.05) (end 130.81 151.13) (width 0.5) (layer B.Cu) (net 10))
 (segment (start 125.73 137.157208) (end 125.73 146.05) (width 0.5) (layer B.Cu) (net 10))
 (segment (start 148.825001 110.889999) (end 149.225 110.49) (width 0.5) (layer B.Cu) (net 10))
 (segment (start 148.825001 130.650336) (end 148.825001 110.889999) (width 0.5) (layer B.Cu) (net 10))
 (segment (start 128.27 135.89) (end 126.997208 135.89) (width 0.5) (layer B.Cu) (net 10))
 (segment (start 140.335 151.13) (end 140.97 150.495) (width 0.5) (layer B.Cu) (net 10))
 (segment (start 130.81 151.13) (end 140.335 151.13) (width 0.5) (layer B.Cu) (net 10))
 (segment (start 126.997208 135.89) (end 125.73 137.157208) (width 0.5) (layer B.Cu) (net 10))
 (segment (start 129.933998 109.22) (end 130.81 108.343998) (width 0.5) (layer B.Cu) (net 13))
 (segment (start 128.27 109.22) (end 129.933998 109.22) (width 0.5) (layer B.Cu) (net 13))
 (segment (start 135.013998 108.343998) (end 135.89 109.22) (width 0.5) (layer B.Cu) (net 13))
 (segment (start 130.81 108.343998) (end 135.013998 108.343998) (width 0.5) (layer B.Cu) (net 13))
 (segment (start 135.89 104.14) (end 135.89 106.68) (width 0.5) (layer B.Cu) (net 13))
 (segment (start 135.89 106.68) (end 135.89 109.22) (width 0.5) (layer B.Cu) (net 13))
 (segment (start 135.89 109.22) (end 135.89 111.76) (width 0.5) (layer B.Cu) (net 13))
 (segment (start 143.51 105.41) (end 143.51 104.14) (width 0.5) (layer B.Cu) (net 22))
 (segment (start 143.51 106.68) (end 143.51 105.41) (width 0.5) (layer B.Cu) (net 22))
 (segment (start 145.415 105.41) (end 143.51 105.41) (width 0.5) (layer B.Cu) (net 22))
 (segment (start 145.560001 105.264999) (end 145.415 105.41) (width 0.5) (layer B.Cu) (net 22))
 (segment (start 145.560001 105.264999) (end 145.560001 128.759999) (width 0.5) (layer B.Cu) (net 22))
 (segment (start 143.51 129.54) (end 143.51 130.81) (width 0.5) (layer B.Cu) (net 22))
 (segment (start 144.78 129.54) (end 143.51 129.54) (width 0.5) (layer B.Cu) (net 22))
 (segment (start 145.560001 128.759999) (end 144.78 129.54) (width 0.5) (layer B.Cu) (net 22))
 (segment (start 143.51 128.27) (end 143.51 129.54) (width 0.5) (layer B.Cu) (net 22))
 (segment (start 145.415 105.119998) (end 145.560001 105.264999) (width 0.5) (layer B.Cu) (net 22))
 (segment (start 129.074324 80.56501) (end 133.138325 80.56501) (width 0.5) (layer B.Cu) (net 22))
 (segment (start 133.839999 79.025999) (end 134.905999 77.959999) (width 0.5) (layer B.Cu) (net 22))
 (segment (start 126.119999 83.519335) (end 129.074324 80.56501) (width 0.5) (layer B.Cu) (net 22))
 (segment (start 145.310001 77.959999) (end 145.560001 78.209999) (width 0.5) (layer B.Cu) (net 22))
 (segment (start 145.560001 100.044001) (end 145.415 100.189002) (width 0.5) (layer B.Cu) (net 22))
 (segment (start 128.27 87.63) (end 126.997208 87.63) (width 0.5) (layer B.Cu) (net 22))
 (segment (start 145.560001 78.209999) (end 145.560001 100.044001) (width 0.5) (layer B.Cu) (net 22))
 (segment (start 134.905999 77.959999) (end 145.310001 77.959999) (width 0.5) (layer B.Cu) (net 22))
 (segment (start 133.138325 80.56501) (end 133.839999 79.863336) (width 0.5) (layer B.Cu) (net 22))
 (segment (start 145.415 100.189002) (end 145.415 105.119998) (width 0.5) (layer B.Cu) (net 22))
 (segment (start 126.997208 87.63) (end 126.119999 86.752791) (width 0.5) (layer B.Cu) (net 22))
 (segment (start 126.119999 86.752791) (end 126.119999 83.519335) (width 0.5) (layer B.Cu) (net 22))
 (segment (start 133.839999 79.863336) (end 133.839999 79.025999) (width 0.5) (layer B.Cu) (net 22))
 (segment (start 135.89 133.35) (end 135.89 130.81) (width 0.5) (layer B.Cu) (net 7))
 (segment (start 135.89 130.81) (end 135.89 128.27) (width 0.5) (layer B.Cu) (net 7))
 (segment (start 135.89 133.35) (end 135.89 135.89) (width 0.5) (layer B.Cu) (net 7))
 (segment (start 128.27 133.35) (end 129.54 132.08) (width 0.5) (layer B.Cu) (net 7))
 (segment (start 129.54 132.08) (end 135.89 132.08) (width 0.5) (layer B.Cu) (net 7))
 (segment (start 135.89 91.44) (end 135.89 93.98) (width 0.5) (layer B.Cu) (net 6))
 (segment (start 135.89 93.98) (end 135.89 96.52) (width 0.5) (layer B.Cu) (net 6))
 (segment (start 135.89 96.52) (end 135.89 99.06) (width 0.5) (layer B.Cu) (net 6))
 (segment (start 132.082792 86.36) (end 130.81 86.36) (width 0.5) (layer B.Cu) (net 6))
 (segment (start 133.839999 88.117207) (end 132.082792 86.36) (width 0.5) (layer B.Cu) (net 6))
 (segment (start 133.839999 89.389999) (end 133.839999 88.117207) (width 0.5) (layer B.Cu) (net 6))
 (segment (start 135.89 91.44) (end 133.839999 89.389999) (width 0.5) (layer B.Cu) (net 6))
 (segment (start 143.51 92.71) (end 143.51 91.44) (width 0.5) (layer F.Cu) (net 1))
 (segment (start 143.51 92.71) (end 143.51 93.98) (width 0.5) (layer F.Cu) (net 1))
 (segment (start 143.51 144.78) (end 143.51 146.05) (width 0.5) (layer F.Cu) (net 1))
 (segment (start 143.51 146.05) (end 143.51 147.32) (width 0.5) (layer F.Cu) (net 1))
 (segment (start 143.51 146.05) (end 149.86 139.7) (width 0.5) (layer F.Cu) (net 1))
 (segment (start 149.86 139.7) (end 149.86 135.185685) (width 0.5) (layer F.Cu) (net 1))
 (segment (start 149.86 135.185685) (end 149.86 134.62) (width 0.5) (layer F.Cu) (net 1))
 (via (at 149.86 134.62) (size 1.6) (drill 0.8) (layers F.Cu B.Cu) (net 1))
 (via (at 136.524992 125.73) (size 1.6) (drill 0.8) (layers F.Cu B.Cu) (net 1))
 (segment (start 133.35 116.837208) (end 133.35 124.390685) (width 0.5) (layer B.Cu) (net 1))
 (segment (start 133.35 124.390685) (end 134.689315 125.73) (width 0.5) (layer B.Cu) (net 1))
 (segment (start 130.81 115.57) (end 132.082792 115.57) (width 0.5) (layer B.Cu) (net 1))
 (segment (start 135.959307 125.73) (end 136.524992 125.73) (width 0.5) (layer B.Cu) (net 1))
 (segment (start 132.082792 115.57) (end 133.35 116.837208) (width 0.5) (layer B.Cu) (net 1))
 (segment (start 134.689315 125.73) (end 135.959307 125.73) (width 0.5) (layer B.Cu) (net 1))
 (segment (start 136.524992 125.73) (end 137.090677 125.73) (width 0.5) (layer F.Cu) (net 1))
 (segment (start 149.86 134.62) (end 152.4 132.08) (width 0.5) (layer B.Cu) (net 1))
 (segment (start 137.090677 125.73) (end 152.4 125.73) (width 0.5) (layer F.Cu) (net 1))
 (segment (start 152.4 132.08) (end 152.4 126.295685) (width 0.5) (layer B.Cu) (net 1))
 (segment (start 152.4 126.295685) (end 152.4 125.73) (width 0.5) (layer B.Cu) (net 1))
 (via (at 152.4 125.73) (size 1.6) (drill 0.8) (layers F.Cu B.Cu) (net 1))
 (via (at 152.545009 93.98) (size 1.6) (drill 0.8) (layers F.Cu B.Cu) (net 1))
 (segment (start 143.51 92.71) (end 144.78 93.98) (width 0.5) (layer F.Cu) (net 1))
 (segment (start 144.78 93.98) (end 151.979324 93.98) (width 0.5) (layer F.Cu) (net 1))
 (segment (start 151.979324 93.98) (end 152.545009 93.98) (width 0.5) (layer F.Cu) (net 1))
 (segment (start 152.654 125.476) (end 152.654 94.088991) (width 0.5) (layer B.Cu) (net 1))
 (segment (start 152.654 94.088991) (end 152.545009 93.98) (width 0.5) (layer B.Cu) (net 1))
 (segment (start 152.4 125.73) (end 152.654 125.476) (width 0.5) (layer B.Cu) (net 1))
 (segment (start 143.51 123.19) (end 143.51 120.65) (width 0.5) (layer B.Cu) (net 4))
 (segment (start 143.51 99.06) (end 143.51 96.52) (width 0.5) (layer B.Cu) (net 4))
 (segment (start 143.51 100.711) (end 143.51 99.06) (width 0.5) (layer B.Cu) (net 4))
 (segment (start 142.710001 123.989999) (end 143.51 123.19) (width 0.5) (layer B.Cu) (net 4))
 (segment (start 142.710001 125.386999) (end 142.710001 123.989999) (width 0.5) (layer B.Cu) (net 4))
 (segment (start 140.843 127.254) (end 142.710001 125.386999) (width 0.5) (layer B.Cu) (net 4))
 (segment (start 141.459999 119.899999) (end 142.21 120.65) (width 0.5) (layer B.Cu) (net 4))
 (segment (start 141.459999 102.761001) (end 141.459999 119.899999) (width 0.5) (layer B.Cu) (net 4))
 (segment (start 142.21 120.65) (end 143.51 120.65) (width 0.5) (layer B.Cu) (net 4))
 (segment (start 143.51 100.711) (end 141.459999 102.761001) (width 0.5) (layer B.Cu) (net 4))
 (segment (start 140.843 146.217002) (end 140.843 127.254) (width 0.5) (layer B.Cu) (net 4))
 (segment (start 137.690001 149.370001) (end 140.843 146.217002) (width 0.5) (layer B.Cu) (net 4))
 (segment (start 134.089999 149.370001) (end 137.690001 149.370001) (width 0.5) (layer B.Cu) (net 4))
 (segment (start 133.839999 149.120001) (end 134.089999 149.370001) (width 0.5) (layer B.Cu) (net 4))
 (segment (start 132.082792 139.7) (end 133.839999 141.457207) (width 0.5) (layer B.Cu) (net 4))
 (segment (start 133.839999 141.457207) (end 133.839999 149.120001) (width 0.5) (layer B.Cu) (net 4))
 (segment (start 130.81 139.7) (end 132.082792 139.7) (width 0.5) (layer B.Cu) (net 4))
 (segment (start 135.89 115.57) (end 135.89 118.11) (width 0.5) (layer B.Cu) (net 5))
 (segment (start 135.89 118.11) (end 135.89 120.65) (width 0.5) (layer B.Cu) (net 5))
 (segment (start 135.89 120.65) (end 135.89 123.19) (width 0.5) (layer B.Cu) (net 5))
 (segment (start 133.839999 112.247207) (end 132.082792 110.49) (width 0.5) (layer B.Cu) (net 5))
 (segment (start 133.839999 113.519999) (end 133.839999 112.247207) (width 0.5) (layer B.Cu) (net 5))
 (segment (start 132.082792 110.49) (end 130.81 110.49) (width 0.5) (layer B.Cu) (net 5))
 (segment (start 135.89 115.57) (end 133.839999 113.519999) (width 0.5) (layer B.Cu) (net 5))
 (segment (start 143.51 115.57) (end 143.51 116.84) (width 0.5) (layer F.Cu) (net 3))
 (segment (start 143.51 116.84) (end 143.51 118.11) (width 0.5) (layer F.Cu) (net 3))
 (segment (start 143.51 139.7) (end 143.51 140.97) (width 0.5) (layer F.Cu) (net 3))
 (segment (start 143.51 140.97) (end 143.51 142.24) (width 0.5) (layer F.Cu) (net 3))
 (via (at 150.495 116.84) (size 1.6) (drill 0.8) (layers F.Cu B.Cu) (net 3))
 (segment (start 143.51 116.84) (end 150.495 116.84) (width 0.5) (layer F.Cu) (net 3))
 (segment (start 150.495 131.44191) (end 148.100009 133.836901) (width 0.5) (layer B.Cu) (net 3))
 (segment (start 148.100009 133.836901) (end 147.70001 134.2369) (width 0.5) (layer B.Cu) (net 3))
 (via (at 147.70001 134.2369) (size 1.6) (drill 0.8) (layers F.Cu B.Cu) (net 3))
 (segment (start 147.70001 136.77999) (end 147.70001 134.802585) (width 0.5) (layer F.Cu) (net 3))
 (segment (start 143.51 140.97) (end 147.70001 136.77999) (width 0.5) (layer F.Cu) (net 3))
 (segment (start 150.495 116.84) (end 150.495 131.44191) (width 0.5) (layer B.Cu) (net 3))
 (segment (start 147.70001 134.802585) (end 147.70001 134.2369) (width 0.5) (layer F.Cu) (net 3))
 (segment (start 150.894999 116.440001) (end 150.495 116.84) (width 0.5) (layer B.Cu) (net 3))
 (segment (start 147.060012 79.49601) (end 150.894999 83.330999) (width 0.5) (layer B.Cu) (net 3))
 (segment (start 132.339988 78.404675) (end 134.284675 76.459988) (width 0.5) (layer B.Cu) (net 3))
 (segment (start 132.339988 78.480012) (end 132.339988 78.404675) (width 0.5) (layer B.Cu) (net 3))
 (segment (start 131.755001 79.064999) (end 132.339988 78.480012) (width 0.5) (layer B.Cu) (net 3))
 (segment (start 132.120023 96.130001) (end 128.507999 96.130001) (width 0.5) (layer B.Cu) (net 3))
 (segment (start 134.284675 76.459988) (end 145.931325 76.459988) (width 0.5) (layer B.Cu) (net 3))
 (segment (start 133.839999 94.410025) (end 132.120023 96.130001) (width 0.5) (layer B.Cu) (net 3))
 (segment (start 133.839999 93.197207) (end 133.839999 94.410025) (width 0.5) (layer B.Cu) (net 3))
 (segment (start 145.931325 76.459988) (end 147.060012 77.588675) (width 0.5) (layer B.Cu) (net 3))
 (segment (start 130.81 91.44) (end 132.082792 91.44) (width 0.5) (layer B.Cu) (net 3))
 (segment (start 147.060012 77.588675) (end 147.060012 79.49601) (width 0.5) (layer B.Cu) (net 3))
 (segment (start 132.082792 91.44) (end 133.839999 93.197207) (width 0.5) (layer B.Cu) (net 3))
 (segment (start 150.894999 83.330999) (end 150.894999 116.440001) (width 0.5) (layer B.Cu) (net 3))
 (segment (start 128.507999 96.130001) (end 116.169999 83.792001) (width 0.5) (layer B.Cu) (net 3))
 (segment (start 116.169999 83.792001) (end 116.169999 80.468999) (width 0.5) (layer B.Cu) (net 3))
 (segment (start 116.169999 80.468999) (end 117.573999 79.064999) (width 0.5) (layer B.Cu) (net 3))
 (segment (start 117.573999 79.064999) (end 131.755001 79.064999) (width 0.5) (layer B.Cu) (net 3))
 (segment (start 135.89 139.7) (end 135.89 142.24) (width 0.5) (layer B.Cu) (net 2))
 (segment (start 135.89 142.24) (end 135.89 144.78) (width 0.5) (layer B.Cu) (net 2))
 (segment (start 135.89 144.78) (end 135.89 147.32) (width 0.5) (layer B.Cu) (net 2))
 (segment (start 135.739991 138.277199) (end 135.739991 139.7) (width 0.5) (layer B.Cu) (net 2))
 (segment (start 135.402793 137.940001) (end 135.739991 138.277199) (width 0.5) (layer B.Cu) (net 2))
 (segment (start 134.089999 137.940001) (end 135.402793 137.940001) (width 0.5) (layer B.Cu) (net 2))
 (segment (start 130.81 134.62) (end 132.082792 134.62) (width 0.5) (layer B.Cu) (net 2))
 (segment (start 133.839999 136.377207) (end 133.839999 137.690001) (width 0.5) (layer B.Cu) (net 2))
 (segment (start 132.082792 134.62) (end 133.839999 136.377207) (width 0.5) (layer B.Cu) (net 2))
 (segment (start 133.839999 137.690001) (end 134.089999 137.940001) (width 0.5) (layer B.Cu) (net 2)))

